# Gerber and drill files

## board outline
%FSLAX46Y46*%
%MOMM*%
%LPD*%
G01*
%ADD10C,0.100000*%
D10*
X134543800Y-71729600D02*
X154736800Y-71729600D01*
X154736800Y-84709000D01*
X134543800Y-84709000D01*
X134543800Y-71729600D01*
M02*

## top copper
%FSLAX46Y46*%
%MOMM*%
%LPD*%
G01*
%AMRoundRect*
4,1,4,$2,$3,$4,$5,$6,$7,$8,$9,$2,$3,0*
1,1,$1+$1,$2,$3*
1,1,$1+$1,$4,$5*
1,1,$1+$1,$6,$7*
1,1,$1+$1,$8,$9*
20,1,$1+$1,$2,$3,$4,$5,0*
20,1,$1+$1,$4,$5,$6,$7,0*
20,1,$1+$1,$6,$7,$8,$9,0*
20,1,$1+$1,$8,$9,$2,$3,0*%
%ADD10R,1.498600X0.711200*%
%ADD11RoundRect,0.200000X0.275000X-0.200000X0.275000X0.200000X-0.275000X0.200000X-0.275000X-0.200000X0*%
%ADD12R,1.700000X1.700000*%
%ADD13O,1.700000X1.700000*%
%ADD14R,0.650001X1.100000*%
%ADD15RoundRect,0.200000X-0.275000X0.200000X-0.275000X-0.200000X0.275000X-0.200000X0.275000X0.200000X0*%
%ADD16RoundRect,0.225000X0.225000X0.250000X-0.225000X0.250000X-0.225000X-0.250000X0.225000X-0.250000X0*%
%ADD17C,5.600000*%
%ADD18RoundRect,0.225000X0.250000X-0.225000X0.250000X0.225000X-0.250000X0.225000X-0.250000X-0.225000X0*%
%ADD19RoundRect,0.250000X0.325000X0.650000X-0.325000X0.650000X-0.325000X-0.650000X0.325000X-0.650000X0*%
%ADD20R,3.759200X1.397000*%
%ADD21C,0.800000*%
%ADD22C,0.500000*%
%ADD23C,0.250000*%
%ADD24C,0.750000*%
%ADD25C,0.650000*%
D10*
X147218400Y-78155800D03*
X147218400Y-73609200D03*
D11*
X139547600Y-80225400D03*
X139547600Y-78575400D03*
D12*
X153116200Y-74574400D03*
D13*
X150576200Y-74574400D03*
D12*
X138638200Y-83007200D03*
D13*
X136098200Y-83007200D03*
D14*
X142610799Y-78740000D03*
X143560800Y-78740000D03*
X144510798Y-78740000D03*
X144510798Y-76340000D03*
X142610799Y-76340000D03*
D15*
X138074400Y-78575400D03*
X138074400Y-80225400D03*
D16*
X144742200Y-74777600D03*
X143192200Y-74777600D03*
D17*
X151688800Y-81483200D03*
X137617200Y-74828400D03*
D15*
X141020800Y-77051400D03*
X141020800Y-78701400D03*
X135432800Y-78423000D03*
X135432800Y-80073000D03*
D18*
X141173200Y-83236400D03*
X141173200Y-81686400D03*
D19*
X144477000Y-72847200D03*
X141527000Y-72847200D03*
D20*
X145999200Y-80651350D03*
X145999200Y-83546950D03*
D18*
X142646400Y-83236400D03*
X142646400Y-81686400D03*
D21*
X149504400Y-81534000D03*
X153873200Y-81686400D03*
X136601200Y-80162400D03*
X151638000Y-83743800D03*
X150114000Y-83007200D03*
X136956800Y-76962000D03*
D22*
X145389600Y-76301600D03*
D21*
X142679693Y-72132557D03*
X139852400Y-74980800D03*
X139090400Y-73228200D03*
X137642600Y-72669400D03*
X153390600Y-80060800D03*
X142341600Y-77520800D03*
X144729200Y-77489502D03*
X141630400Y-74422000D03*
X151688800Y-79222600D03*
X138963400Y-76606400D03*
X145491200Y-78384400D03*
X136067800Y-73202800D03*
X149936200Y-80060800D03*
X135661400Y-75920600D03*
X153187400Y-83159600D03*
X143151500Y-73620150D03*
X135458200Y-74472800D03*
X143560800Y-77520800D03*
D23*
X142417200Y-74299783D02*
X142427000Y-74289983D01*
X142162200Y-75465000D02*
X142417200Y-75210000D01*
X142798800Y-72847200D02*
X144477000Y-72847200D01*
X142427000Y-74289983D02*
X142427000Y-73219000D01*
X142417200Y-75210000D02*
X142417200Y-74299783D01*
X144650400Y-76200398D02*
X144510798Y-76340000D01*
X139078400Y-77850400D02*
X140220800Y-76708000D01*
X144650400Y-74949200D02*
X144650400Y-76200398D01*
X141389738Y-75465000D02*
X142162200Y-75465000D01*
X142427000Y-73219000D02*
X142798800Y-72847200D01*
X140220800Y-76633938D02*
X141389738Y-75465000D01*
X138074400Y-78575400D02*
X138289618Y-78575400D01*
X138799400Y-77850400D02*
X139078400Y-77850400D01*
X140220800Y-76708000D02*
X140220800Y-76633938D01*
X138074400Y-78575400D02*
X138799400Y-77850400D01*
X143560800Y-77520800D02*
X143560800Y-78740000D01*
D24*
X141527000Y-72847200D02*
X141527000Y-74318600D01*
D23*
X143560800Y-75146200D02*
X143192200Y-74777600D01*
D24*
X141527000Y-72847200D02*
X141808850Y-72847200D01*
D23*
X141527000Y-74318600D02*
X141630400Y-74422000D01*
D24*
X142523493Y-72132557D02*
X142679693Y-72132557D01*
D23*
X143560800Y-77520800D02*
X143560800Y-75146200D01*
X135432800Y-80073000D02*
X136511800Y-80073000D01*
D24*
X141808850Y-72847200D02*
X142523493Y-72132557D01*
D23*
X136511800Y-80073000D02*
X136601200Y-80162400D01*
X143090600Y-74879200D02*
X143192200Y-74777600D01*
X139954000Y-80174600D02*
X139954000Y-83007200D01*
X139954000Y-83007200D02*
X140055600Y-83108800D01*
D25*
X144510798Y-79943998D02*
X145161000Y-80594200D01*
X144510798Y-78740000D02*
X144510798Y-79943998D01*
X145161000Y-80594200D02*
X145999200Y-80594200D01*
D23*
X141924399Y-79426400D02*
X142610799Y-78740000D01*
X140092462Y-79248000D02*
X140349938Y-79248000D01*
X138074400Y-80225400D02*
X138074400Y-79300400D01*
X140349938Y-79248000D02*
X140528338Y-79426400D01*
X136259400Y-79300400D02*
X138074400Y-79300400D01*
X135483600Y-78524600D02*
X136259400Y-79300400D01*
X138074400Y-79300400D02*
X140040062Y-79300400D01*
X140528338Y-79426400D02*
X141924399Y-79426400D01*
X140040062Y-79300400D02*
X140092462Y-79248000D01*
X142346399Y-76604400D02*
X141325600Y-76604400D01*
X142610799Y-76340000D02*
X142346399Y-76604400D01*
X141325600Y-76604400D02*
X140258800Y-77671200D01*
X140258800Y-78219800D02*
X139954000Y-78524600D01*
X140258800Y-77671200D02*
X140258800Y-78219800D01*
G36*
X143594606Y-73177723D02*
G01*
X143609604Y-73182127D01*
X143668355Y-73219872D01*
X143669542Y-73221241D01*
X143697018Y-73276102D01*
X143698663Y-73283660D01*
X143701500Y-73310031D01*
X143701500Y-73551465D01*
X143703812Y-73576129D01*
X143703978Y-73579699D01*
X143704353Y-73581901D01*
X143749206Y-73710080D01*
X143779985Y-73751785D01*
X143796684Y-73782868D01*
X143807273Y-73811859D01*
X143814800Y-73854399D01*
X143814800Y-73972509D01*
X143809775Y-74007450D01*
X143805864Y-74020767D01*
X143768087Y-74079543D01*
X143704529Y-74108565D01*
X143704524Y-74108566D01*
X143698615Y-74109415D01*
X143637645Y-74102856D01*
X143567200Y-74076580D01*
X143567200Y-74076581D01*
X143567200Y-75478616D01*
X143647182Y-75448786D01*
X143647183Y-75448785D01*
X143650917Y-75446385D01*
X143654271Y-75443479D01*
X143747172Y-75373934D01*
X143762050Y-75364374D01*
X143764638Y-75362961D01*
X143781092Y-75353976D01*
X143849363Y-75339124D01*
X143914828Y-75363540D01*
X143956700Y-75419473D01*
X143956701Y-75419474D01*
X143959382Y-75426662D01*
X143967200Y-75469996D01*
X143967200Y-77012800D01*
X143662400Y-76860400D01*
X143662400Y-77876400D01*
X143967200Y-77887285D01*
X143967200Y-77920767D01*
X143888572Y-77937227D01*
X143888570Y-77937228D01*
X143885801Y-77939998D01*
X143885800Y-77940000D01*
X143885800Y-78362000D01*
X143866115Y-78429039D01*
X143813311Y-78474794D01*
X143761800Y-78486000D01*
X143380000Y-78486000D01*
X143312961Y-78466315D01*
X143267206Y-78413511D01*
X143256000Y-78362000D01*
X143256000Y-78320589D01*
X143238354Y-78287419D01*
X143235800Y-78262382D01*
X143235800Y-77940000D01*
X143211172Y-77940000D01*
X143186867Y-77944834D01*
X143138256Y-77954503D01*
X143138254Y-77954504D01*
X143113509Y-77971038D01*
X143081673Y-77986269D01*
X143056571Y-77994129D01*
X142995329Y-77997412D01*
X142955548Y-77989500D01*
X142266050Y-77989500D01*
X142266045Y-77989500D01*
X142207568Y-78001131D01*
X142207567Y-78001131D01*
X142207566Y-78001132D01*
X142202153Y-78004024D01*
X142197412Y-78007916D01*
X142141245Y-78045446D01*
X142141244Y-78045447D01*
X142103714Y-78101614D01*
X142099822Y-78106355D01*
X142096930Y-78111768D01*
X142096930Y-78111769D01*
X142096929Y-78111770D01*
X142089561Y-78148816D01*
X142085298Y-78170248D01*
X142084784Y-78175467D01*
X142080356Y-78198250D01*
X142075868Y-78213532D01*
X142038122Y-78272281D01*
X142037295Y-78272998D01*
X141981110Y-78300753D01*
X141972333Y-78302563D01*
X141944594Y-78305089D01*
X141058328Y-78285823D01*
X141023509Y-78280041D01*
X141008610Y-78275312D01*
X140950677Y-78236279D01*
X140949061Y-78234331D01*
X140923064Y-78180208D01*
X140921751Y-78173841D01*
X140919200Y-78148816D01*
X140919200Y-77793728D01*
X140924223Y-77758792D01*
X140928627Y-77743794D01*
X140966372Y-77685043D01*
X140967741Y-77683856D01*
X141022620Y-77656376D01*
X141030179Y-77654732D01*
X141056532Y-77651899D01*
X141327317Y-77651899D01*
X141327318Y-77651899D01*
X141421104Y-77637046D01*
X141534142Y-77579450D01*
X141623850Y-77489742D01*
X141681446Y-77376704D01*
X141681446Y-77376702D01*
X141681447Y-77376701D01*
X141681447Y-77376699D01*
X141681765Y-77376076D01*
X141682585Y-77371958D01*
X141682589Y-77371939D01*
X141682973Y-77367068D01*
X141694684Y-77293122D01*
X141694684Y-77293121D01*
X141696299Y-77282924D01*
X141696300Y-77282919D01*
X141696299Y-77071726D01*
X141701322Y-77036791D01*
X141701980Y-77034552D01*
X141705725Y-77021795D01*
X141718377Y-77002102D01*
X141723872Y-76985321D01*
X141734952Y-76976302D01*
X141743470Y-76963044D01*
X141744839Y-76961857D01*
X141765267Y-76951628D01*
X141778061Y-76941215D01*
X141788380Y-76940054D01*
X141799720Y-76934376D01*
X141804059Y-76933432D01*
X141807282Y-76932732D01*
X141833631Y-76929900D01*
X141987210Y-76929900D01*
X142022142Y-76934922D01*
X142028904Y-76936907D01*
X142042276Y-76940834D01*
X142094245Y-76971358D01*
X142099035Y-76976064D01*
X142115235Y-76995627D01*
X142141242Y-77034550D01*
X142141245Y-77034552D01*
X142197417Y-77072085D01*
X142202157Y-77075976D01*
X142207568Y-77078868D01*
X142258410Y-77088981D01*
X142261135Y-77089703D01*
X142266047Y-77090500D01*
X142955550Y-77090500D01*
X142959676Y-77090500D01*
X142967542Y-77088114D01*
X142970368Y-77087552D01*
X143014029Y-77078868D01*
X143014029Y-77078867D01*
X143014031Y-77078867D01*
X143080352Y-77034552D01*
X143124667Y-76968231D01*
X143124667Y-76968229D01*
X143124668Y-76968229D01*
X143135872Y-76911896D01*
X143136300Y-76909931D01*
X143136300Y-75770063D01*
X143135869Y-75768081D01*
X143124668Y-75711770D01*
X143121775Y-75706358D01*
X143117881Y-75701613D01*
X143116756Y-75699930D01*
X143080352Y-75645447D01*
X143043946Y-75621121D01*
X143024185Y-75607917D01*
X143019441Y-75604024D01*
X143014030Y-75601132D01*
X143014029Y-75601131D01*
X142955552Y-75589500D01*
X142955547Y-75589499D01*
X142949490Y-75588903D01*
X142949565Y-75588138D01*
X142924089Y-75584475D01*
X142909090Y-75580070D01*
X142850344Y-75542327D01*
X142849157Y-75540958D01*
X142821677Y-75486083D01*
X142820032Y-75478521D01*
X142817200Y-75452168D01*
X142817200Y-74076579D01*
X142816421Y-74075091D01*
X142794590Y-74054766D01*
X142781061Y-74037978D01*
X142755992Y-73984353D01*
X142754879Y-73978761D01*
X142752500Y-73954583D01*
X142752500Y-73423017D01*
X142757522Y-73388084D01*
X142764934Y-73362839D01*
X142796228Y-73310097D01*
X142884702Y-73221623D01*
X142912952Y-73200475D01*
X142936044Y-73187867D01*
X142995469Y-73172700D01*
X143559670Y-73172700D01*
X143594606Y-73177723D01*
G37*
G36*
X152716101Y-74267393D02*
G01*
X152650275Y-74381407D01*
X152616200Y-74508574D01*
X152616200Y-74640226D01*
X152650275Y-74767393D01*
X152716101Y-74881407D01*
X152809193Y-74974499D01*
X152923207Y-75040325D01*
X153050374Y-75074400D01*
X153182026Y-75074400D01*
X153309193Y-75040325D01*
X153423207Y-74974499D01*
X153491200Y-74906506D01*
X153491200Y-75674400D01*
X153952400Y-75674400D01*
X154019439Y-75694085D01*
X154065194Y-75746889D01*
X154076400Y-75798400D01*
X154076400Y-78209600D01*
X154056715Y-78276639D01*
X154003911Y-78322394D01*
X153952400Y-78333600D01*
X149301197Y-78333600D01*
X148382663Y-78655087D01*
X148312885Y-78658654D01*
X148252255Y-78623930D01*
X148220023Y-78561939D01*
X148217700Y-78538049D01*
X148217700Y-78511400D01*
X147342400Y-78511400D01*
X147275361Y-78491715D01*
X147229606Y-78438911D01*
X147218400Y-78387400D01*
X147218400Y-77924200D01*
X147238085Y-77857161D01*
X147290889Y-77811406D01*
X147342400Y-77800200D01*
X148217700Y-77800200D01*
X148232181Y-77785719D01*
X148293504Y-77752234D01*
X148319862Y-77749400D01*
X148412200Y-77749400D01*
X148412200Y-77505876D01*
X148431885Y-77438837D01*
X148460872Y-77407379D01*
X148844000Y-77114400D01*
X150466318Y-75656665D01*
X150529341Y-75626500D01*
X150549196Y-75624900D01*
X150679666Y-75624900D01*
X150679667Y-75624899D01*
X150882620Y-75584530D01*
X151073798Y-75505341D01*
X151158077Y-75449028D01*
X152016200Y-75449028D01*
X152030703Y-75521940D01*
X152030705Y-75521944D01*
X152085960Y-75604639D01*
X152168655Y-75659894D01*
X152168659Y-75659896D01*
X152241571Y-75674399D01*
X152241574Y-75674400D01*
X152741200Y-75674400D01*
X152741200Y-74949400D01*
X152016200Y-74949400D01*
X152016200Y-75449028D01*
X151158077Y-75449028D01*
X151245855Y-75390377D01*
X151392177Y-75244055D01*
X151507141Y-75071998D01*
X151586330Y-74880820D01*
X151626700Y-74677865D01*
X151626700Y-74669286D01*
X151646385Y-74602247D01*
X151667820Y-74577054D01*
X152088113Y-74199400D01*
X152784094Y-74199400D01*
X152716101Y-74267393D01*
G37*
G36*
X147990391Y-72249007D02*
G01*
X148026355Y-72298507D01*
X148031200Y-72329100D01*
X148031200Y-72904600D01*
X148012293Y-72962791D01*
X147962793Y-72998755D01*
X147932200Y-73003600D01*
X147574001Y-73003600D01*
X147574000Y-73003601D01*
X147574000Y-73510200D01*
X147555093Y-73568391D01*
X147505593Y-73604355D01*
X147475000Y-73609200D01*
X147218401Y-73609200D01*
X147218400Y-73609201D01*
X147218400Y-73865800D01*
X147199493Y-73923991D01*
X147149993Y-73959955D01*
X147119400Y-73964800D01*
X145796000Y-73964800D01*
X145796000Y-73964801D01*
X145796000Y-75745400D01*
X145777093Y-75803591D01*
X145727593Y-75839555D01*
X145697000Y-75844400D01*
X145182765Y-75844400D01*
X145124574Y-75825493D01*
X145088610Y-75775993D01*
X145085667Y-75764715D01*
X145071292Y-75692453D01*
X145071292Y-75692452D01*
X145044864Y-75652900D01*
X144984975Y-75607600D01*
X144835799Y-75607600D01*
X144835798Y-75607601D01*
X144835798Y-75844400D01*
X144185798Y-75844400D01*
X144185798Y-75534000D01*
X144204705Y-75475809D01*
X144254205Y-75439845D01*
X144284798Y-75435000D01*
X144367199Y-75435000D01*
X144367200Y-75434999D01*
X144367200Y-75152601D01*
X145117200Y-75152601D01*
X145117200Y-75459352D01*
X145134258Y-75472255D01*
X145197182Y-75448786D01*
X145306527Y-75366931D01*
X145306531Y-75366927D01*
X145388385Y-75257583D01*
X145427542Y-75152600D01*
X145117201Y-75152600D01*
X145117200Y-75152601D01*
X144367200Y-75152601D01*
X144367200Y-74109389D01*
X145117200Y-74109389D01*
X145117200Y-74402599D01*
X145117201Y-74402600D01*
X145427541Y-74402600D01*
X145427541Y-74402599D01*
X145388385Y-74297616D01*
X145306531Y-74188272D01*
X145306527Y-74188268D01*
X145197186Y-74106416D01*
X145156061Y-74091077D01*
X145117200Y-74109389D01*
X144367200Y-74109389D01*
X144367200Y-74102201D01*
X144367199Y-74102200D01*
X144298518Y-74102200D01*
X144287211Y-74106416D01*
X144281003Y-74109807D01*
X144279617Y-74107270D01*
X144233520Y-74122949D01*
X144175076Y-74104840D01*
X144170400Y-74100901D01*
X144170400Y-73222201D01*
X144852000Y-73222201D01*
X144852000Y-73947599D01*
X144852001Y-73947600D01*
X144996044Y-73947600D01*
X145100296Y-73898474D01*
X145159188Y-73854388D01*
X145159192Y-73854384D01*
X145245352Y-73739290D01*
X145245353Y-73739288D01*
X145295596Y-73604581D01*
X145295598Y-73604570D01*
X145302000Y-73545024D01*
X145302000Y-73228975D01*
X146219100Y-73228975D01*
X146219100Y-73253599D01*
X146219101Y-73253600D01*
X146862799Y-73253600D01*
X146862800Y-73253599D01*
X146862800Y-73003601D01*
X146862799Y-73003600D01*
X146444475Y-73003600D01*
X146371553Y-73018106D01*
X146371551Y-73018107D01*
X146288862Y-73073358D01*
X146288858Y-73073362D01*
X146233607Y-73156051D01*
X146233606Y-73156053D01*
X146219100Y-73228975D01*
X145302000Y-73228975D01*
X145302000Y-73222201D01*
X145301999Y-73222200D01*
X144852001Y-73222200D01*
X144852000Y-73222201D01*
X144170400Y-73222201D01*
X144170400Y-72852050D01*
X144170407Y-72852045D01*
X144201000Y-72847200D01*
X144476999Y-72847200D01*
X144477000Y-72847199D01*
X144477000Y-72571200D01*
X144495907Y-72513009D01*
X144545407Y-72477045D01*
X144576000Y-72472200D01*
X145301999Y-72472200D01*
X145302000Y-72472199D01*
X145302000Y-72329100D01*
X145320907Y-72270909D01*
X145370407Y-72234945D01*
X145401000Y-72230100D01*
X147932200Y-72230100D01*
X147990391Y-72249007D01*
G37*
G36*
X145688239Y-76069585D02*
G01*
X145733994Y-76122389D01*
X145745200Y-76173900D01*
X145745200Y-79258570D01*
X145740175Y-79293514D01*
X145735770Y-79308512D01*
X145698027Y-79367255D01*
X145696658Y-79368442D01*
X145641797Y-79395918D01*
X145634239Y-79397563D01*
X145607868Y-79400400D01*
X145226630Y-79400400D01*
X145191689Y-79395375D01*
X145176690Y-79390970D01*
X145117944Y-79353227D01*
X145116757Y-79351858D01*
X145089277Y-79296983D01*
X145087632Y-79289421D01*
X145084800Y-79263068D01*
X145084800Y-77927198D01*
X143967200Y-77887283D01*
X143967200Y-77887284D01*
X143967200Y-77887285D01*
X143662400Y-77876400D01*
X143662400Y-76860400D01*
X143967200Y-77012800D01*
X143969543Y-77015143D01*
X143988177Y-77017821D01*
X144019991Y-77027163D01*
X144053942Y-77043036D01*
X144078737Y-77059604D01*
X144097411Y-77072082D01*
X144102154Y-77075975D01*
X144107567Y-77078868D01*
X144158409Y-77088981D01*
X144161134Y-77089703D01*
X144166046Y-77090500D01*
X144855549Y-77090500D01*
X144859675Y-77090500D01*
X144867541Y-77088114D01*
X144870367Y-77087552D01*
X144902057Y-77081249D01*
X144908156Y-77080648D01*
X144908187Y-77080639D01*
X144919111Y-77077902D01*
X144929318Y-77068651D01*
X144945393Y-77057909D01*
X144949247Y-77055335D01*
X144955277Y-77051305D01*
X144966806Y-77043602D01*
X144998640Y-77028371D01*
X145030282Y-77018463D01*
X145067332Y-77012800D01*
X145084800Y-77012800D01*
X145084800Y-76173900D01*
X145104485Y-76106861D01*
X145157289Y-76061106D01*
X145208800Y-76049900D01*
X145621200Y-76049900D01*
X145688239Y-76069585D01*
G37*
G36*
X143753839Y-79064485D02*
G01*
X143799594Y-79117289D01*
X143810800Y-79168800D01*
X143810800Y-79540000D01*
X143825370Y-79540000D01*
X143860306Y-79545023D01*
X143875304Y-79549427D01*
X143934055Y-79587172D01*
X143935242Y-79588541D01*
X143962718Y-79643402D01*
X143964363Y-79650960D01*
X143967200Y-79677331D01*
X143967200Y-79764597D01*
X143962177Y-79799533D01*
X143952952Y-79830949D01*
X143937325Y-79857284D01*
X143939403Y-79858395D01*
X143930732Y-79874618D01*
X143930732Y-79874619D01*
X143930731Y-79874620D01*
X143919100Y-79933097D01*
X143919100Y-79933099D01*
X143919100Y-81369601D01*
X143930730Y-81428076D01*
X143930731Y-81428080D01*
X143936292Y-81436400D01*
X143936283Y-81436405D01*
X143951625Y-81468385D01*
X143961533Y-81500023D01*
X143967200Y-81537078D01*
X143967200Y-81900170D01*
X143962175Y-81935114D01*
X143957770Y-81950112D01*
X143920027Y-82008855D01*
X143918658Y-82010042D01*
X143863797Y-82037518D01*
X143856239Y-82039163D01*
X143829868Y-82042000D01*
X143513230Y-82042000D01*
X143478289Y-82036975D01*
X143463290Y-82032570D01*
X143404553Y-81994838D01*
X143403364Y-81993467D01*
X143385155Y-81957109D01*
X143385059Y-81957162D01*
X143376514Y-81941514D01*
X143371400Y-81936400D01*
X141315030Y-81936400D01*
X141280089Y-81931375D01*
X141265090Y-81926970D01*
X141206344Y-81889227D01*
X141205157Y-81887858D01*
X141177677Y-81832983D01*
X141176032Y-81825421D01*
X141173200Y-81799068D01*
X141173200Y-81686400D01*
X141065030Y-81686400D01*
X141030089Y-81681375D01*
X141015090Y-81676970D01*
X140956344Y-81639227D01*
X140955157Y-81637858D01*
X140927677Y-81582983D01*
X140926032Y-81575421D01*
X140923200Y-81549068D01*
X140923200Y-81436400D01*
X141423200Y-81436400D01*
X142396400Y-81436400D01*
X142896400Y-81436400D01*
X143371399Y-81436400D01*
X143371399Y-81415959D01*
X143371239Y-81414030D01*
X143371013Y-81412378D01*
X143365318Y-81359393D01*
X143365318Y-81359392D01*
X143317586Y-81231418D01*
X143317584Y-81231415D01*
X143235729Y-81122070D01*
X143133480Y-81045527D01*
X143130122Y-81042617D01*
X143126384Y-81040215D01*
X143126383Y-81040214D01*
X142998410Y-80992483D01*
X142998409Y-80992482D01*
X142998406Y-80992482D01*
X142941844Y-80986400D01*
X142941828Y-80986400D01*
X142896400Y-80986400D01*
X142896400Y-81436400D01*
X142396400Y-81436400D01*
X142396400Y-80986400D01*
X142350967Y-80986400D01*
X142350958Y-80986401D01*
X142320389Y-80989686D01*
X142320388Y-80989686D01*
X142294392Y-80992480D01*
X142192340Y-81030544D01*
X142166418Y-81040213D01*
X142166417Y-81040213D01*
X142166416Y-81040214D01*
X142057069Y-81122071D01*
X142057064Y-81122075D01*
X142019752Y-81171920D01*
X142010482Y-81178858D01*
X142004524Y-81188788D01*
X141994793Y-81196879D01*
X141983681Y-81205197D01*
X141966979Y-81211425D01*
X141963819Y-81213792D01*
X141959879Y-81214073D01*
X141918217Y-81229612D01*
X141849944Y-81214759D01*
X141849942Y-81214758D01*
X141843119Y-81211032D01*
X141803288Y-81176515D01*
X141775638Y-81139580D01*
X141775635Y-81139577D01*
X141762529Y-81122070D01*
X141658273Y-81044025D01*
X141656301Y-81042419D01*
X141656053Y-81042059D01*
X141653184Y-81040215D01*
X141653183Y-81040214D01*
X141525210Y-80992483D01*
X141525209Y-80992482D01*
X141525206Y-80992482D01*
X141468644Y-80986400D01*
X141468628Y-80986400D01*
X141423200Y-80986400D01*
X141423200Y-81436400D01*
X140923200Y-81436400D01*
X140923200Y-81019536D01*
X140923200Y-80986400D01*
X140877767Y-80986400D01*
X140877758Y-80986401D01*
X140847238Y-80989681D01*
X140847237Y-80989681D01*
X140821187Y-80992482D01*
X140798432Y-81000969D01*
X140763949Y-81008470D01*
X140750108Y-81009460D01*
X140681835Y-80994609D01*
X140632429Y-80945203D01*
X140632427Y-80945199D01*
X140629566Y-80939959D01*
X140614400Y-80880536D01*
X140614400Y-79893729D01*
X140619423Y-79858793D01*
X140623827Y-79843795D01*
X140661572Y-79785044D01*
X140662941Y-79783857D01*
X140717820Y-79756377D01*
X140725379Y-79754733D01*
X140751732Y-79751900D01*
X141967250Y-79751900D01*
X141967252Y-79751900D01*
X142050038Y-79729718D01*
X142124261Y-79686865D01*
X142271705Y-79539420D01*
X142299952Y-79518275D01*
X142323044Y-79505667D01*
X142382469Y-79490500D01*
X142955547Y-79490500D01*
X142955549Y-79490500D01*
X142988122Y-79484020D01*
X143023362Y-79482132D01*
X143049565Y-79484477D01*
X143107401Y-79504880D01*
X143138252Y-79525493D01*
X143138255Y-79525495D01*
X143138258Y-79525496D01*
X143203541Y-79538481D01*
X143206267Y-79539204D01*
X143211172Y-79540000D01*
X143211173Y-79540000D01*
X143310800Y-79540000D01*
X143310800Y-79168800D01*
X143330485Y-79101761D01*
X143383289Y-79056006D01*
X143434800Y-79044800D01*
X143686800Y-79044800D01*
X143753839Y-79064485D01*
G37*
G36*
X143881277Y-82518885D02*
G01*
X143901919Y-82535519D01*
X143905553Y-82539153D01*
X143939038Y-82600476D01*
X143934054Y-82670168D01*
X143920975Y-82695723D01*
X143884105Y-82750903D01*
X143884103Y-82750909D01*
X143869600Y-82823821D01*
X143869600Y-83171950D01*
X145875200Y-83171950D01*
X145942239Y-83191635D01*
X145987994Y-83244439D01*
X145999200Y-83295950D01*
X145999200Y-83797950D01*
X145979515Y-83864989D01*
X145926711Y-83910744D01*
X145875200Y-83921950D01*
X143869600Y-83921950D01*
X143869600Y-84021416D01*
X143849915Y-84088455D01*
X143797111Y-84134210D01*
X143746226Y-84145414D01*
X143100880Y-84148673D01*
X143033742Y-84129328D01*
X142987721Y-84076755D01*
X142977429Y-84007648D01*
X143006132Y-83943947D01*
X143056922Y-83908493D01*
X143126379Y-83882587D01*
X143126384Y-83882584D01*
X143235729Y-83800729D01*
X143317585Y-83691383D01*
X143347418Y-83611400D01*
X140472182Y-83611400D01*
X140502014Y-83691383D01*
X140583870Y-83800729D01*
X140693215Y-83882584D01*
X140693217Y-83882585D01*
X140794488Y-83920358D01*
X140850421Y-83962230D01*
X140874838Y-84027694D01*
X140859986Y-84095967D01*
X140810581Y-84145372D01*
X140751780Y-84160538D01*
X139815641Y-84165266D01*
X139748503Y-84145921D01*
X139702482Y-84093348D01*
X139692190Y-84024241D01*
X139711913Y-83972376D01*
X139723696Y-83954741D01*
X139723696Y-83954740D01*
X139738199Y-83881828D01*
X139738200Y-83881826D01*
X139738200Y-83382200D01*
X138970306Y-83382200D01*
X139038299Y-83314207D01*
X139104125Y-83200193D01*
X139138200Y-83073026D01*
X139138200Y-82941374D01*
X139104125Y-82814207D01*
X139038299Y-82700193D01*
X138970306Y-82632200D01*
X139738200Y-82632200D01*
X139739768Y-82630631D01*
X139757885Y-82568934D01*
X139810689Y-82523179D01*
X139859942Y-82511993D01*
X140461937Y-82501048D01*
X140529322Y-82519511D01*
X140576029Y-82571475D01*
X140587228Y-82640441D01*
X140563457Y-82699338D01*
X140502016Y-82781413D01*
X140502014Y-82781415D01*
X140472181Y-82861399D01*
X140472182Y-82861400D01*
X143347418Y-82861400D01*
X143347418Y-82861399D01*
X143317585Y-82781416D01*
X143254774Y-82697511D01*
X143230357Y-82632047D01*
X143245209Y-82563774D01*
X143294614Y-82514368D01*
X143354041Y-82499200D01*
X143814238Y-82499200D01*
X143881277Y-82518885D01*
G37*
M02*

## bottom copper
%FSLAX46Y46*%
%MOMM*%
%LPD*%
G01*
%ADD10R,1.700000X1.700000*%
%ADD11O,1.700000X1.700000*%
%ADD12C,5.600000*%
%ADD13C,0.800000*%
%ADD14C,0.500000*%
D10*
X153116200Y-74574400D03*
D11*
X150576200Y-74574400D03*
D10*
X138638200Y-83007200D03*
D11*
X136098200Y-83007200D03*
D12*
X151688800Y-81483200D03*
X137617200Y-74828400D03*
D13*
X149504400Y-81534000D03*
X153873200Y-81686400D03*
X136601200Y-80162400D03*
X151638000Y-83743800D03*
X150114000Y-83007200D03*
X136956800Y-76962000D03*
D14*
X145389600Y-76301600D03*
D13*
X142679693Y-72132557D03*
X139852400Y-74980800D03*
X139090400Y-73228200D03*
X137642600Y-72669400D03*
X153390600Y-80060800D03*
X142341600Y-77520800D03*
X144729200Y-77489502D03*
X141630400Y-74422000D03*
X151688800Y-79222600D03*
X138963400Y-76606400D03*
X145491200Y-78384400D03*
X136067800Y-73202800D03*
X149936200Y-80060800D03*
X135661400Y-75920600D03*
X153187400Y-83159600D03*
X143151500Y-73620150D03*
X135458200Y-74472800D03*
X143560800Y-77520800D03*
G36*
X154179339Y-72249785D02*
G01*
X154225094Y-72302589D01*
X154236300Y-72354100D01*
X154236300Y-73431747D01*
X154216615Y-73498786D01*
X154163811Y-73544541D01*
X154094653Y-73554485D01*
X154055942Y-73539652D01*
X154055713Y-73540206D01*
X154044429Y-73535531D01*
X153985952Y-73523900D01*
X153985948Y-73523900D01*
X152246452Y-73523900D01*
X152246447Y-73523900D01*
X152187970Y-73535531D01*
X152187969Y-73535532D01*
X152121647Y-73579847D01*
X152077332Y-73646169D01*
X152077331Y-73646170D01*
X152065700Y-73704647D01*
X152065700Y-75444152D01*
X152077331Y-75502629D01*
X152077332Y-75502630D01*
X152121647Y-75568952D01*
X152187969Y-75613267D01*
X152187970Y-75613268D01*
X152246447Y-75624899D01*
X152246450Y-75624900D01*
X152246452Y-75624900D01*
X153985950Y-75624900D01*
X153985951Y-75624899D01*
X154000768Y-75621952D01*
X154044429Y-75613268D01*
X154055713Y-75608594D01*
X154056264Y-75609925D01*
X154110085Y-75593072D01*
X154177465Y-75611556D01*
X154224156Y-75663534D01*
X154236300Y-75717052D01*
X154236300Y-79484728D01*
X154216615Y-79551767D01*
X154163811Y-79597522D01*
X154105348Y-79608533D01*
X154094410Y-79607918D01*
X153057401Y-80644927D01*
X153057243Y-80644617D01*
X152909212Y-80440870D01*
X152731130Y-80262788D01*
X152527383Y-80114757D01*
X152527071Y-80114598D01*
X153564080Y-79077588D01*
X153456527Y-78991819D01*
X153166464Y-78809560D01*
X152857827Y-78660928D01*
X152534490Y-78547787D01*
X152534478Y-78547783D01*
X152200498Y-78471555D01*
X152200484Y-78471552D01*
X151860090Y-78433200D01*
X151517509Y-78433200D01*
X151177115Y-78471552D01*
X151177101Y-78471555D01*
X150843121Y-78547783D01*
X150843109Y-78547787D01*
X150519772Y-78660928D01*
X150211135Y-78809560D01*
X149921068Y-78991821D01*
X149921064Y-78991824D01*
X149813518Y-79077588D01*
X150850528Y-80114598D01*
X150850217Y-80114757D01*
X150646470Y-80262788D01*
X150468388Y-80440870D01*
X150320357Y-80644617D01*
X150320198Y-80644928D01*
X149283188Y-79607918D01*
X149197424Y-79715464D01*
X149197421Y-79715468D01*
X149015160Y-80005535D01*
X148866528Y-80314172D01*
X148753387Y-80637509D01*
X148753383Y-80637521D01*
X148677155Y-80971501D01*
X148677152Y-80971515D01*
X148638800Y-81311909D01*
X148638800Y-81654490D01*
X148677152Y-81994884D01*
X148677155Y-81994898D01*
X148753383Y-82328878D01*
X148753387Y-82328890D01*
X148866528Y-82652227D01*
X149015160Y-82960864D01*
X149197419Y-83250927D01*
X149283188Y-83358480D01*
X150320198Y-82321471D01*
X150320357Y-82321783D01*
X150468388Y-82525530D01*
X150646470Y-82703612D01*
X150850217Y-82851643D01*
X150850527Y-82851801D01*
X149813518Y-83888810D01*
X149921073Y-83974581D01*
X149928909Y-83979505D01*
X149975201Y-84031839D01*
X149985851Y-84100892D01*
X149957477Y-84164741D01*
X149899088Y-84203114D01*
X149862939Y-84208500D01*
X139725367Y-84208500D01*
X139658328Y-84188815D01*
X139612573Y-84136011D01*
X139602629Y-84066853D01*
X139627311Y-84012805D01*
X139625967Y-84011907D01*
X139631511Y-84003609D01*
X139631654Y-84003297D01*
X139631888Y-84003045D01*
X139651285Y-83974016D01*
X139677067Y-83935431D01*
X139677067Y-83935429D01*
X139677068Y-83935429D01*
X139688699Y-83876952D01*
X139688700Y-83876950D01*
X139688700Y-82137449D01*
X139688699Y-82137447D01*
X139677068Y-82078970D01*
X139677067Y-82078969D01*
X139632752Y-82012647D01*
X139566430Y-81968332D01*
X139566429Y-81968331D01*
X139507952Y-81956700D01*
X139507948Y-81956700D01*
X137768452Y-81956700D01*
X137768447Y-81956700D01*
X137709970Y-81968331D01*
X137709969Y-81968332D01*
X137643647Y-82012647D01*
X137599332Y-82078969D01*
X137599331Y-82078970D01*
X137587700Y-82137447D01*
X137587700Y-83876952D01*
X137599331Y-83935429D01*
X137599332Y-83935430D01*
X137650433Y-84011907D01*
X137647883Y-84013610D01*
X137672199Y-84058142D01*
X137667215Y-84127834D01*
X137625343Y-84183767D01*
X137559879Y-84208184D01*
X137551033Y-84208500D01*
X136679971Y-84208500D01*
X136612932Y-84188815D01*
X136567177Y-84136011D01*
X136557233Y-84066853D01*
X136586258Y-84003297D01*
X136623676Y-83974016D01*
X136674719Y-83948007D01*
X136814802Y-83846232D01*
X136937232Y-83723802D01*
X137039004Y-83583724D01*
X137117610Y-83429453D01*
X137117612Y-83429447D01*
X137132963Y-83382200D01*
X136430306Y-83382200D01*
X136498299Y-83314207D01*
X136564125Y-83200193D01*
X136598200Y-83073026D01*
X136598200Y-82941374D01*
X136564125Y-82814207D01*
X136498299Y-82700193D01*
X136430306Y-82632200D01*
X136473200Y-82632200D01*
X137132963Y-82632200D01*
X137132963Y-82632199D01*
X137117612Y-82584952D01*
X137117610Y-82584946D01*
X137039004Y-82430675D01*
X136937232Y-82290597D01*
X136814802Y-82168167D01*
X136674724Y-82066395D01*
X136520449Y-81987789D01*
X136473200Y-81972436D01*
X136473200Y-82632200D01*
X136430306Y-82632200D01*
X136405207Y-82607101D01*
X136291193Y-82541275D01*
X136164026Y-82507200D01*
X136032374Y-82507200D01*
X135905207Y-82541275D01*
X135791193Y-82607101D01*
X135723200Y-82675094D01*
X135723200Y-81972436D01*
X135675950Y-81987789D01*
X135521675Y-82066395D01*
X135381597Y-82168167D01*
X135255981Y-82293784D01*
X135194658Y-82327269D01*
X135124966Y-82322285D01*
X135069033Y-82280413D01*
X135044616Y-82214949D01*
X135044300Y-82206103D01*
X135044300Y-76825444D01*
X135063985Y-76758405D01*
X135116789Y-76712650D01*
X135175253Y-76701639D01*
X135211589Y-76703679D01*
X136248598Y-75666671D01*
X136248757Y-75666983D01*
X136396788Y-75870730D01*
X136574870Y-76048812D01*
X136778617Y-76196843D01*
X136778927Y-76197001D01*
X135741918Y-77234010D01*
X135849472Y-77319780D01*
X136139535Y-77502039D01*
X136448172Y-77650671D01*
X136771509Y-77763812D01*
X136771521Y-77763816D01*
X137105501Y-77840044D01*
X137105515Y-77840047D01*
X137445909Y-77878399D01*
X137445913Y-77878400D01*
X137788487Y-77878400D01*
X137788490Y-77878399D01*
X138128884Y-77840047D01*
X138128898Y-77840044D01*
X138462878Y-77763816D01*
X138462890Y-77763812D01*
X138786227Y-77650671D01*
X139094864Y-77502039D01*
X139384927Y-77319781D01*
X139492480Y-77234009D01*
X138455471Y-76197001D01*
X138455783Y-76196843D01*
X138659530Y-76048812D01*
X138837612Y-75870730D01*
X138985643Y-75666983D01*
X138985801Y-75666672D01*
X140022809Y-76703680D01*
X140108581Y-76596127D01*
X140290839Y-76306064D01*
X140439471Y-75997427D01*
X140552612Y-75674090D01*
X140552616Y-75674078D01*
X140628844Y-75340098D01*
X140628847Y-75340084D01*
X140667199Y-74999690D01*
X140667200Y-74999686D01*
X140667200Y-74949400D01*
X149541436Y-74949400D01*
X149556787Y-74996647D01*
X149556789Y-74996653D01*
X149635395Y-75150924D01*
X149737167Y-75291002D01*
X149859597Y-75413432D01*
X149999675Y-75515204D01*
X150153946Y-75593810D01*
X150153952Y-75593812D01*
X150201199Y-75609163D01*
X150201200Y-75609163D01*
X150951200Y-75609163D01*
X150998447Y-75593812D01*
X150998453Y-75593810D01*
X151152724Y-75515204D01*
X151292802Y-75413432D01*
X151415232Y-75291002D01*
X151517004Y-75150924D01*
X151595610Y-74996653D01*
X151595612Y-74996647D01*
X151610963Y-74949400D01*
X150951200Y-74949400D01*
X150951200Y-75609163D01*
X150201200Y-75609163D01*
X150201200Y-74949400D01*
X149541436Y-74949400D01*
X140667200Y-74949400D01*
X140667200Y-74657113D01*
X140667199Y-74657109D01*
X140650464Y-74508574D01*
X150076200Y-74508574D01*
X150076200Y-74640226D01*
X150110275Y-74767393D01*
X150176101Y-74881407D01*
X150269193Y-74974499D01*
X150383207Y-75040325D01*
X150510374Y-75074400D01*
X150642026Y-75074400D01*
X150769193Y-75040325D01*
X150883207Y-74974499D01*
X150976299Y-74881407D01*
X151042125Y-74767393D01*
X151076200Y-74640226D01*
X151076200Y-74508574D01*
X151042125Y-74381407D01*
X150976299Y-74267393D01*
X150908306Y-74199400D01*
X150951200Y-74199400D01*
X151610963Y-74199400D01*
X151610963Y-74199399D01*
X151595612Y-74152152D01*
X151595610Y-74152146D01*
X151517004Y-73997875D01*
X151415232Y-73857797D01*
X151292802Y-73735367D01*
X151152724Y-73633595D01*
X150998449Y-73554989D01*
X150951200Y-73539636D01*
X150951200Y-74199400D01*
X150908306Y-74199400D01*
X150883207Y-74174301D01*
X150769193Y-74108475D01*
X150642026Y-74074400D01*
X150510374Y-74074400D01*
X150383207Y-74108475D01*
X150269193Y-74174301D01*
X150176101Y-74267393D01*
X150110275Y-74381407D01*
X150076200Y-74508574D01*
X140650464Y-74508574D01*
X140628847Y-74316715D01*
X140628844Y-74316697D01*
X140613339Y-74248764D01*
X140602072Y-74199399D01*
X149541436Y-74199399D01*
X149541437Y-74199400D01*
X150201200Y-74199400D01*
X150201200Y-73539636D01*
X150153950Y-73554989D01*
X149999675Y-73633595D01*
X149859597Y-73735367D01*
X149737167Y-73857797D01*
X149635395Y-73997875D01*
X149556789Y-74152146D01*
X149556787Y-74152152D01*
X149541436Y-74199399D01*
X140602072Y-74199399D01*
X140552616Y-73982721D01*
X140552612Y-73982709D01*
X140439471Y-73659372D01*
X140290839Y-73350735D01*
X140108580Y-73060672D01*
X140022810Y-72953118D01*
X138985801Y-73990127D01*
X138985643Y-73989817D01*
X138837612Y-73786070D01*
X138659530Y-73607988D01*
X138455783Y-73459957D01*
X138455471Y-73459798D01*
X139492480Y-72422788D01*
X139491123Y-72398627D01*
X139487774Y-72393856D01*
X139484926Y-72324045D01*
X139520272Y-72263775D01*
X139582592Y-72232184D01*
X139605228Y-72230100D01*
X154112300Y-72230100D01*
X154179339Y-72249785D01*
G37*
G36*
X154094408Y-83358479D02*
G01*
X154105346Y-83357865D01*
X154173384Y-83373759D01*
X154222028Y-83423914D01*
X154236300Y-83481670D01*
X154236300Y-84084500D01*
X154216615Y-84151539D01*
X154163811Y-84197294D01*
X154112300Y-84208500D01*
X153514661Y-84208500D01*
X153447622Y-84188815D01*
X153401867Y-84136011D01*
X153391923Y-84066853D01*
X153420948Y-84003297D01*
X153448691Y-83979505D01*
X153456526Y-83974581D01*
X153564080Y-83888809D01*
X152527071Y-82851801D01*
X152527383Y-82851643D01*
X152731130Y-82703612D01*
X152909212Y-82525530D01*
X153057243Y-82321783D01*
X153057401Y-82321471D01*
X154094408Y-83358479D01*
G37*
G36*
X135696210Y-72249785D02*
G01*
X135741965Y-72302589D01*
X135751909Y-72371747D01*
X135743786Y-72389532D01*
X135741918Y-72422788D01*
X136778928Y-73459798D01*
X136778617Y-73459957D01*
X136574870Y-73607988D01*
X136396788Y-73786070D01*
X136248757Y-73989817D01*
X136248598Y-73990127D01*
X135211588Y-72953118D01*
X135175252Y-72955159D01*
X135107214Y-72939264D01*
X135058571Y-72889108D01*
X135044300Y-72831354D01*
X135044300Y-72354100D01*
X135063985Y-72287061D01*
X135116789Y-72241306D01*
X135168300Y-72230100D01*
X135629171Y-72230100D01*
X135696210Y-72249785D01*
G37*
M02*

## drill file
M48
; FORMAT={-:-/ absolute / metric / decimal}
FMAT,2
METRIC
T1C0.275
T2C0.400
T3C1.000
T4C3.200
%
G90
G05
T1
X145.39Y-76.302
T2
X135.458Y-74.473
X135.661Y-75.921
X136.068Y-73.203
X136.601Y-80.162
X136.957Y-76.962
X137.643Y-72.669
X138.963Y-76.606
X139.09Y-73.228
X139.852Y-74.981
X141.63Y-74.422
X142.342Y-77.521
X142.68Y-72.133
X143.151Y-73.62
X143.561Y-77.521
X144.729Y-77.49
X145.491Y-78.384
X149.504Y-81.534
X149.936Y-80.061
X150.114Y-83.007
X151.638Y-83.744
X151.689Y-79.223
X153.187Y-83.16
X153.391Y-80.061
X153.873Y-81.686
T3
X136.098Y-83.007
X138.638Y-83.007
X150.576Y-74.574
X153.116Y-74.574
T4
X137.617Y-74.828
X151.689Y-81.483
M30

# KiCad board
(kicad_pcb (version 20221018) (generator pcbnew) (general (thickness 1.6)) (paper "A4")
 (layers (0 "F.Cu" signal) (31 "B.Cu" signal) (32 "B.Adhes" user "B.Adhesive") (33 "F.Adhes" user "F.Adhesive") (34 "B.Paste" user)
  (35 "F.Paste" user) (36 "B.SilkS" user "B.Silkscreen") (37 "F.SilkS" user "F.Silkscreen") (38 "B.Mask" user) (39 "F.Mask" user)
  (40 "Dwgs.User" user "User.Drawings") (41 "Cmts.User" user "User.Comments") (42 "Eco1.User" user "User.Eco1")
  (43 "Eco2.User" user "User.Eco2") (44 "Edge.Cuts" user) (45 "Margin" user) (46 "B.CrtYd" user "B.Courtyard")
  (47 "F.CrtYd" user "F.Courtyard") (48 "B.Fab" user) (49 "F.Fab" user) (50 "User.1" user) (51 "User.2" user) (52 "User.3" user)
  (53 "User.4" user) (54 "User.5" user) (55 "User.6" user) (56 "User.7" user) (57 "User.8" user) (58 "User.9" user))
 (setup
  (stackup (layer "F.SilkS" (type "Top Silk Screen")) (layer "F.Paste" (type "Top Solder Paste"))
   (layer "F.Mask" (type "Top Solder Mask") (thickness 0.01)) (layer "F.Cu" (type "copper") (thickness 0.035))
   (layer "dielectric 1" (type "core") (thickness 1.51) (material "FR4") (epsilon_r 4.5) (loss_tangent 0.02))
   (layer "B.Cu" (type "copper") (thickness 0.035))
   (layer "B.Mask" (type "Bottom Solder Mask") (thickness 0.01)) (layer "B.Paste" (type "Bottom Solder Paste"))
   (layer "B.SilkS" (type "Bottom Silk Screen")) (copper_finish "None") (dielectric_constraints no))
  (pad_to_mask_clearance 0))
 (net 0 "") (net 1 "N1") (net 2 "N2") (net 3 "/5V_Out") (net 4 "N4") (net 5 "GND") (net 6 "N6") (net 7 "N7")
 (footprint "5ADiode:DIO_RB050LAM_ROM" (layer "F.Cu") (at 147.2184 75.8825 90)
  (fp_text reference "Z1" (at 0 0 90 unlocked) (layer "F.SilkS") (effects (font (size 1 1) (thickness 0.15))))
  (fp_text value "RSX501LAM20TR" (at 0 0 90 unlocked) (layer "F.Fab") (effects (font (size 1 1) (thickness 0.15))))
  (pad "1" smd rect (at -2.2733 0 90) (size 0.7112 1.4986) (layers "F.Cu" "F.Paste" "F.Mask") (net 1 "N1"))
  (pad "2" smd rect (at 2.2733 0 90) (size 0.7112 1.4986) (layers "F.Cu" "F.Paste" "F.Mask") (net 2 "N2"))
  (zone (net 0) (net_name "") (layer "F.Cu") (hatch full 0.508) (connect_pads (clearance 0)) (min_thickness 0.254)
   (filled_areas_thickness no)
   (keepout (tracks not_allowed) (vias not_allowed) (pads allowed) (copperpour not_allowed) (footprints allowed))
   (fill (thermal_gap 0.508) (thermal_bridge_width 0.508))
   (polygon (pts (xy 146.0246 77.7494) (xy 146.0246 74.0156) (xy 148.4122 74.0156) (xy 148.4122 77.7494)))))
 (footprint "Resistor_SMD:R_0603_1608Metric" (layer "F.Cu") (at 139.5476 79.4004 90)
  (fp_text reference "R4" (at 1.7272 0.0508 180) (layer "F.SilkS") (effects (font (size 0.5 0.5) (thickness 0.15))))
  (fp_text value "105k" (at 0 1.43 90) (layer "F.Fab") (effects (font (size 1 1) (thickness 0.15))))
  (pad "1" smd roundrect (at -0.825 0 90) (size 0.8 0.95) (layers "F.Cu" "F.Paste" "F.Mask") (roundrect_rratio 0.25) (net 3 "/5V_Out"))
  (pad "2" smd roundrect (at 0.825 0 90) (size 0.8 0.95) (layers "F.Cu" "F.Paste" "F.Mask") (roundrect_rratio 0.25) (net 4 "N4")))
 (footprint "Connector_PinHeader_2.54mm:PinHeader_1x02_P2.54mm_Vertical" (layer "F.Cu") (at 153.1162 74.5744 -90)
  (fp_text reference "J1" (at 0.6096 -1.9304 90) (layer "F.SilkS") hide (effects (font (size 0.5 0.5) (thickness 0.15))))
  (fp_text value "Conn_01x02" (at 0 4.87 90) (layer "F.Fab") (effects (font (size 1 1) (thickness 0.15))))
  (pad "1" thru_hole rect (at 0 0 270) (size 1.7 1.7) (drill 1) (layers "*.Cu" "*.Mask") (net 1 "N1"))
  (pad "2" thru_hole oval (at 0 2.54 270) (size 1.7 1.7) (drill 1) (layers "*.Cu" "*.Mask") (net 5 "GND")))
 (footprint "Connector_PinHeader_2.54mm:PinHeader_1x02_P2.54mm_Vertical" (layer "F.Cu") (at 138.6382 83.0072 -90)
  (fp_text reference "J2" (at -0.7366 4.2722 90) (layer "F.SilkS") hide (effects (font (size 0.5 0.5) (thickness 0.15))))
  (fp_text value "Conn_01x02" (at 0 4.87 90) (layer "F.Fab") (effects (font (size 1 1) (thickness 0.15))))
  (pad "1" thru_hole rect (at 0 0 270) (size 1.7 1.7) (drill 1) (layers "*.Cu" "*.Mask") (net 3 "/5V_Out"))
  (pad "2" thru_hole oval (at 0 2.54 270) (size 1.7 1.7) (drill 1) (layers "*.Cu" "*.Mask") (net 5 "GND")))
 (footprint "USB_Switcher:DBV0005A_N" (layer "F.Cu") (at 143.5608 77.54 90)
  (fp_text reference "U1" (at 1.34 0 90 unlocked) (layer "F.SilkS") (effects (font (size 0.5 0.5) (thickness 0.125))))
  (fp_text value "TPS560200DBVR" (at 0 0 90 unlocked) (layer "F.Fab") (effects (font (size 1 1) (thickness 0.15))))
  (pad "1" smd rect (at -1.2 -0.950001 180) (size 0.650001 1.1) (layers "F.Cu" "F.Paste" "F.Mask") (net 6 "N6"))
  (pad "2" smd rect (at -1.2 0 180) (size 0.650001 1.1) (layers "F.Cu" "F.Paste" "F.Mask") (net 5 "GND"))
  (pad "3" smd rect (at -1.2 0.949998 180) (size 0.650001 1.1) (layers "F.Cu" "F.Paste" "F.Mask") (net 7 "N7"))
  (pad "4" smd rect (at 1.2 0.949998 180) (size 0.650001 1.1) (layers "F.Cu" "F.Paste" "F.Mask") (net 2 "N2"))
  (pad "5" smd rect (at 1.2 -0.950001 180) (size 0.650001 1.1) (layers "F.Cu" "F.Paste" "F.Mask") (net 4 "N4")))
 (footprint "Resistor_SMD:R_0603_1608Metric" (layer "F.Cu") (at 138.0744 79.4004 -90)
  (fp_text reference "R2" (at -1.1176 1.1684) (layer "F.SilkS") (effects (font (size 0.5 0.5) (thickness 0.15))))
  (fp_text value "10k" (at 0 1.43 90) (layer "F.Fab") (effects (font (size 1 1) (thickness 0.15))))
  (pad "1" smd roundrect (at -0.825 0 270) (size 0.8 0.95) (layers "F.Cu" "F.Paste" "F.Mask") (roundrect_rratio 0.25) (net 2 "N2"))
  (pad "2" smd roundrect (at 0.825 0 270) (size 0.8 0.95) (layers "F.Cu" "F.Paste" "F.Mask") (roundrect_rratio 0.25) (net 6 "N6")))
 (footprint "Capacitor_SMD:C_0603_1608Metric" (layer "F.Cu") (at 143.9672 74.7776 180)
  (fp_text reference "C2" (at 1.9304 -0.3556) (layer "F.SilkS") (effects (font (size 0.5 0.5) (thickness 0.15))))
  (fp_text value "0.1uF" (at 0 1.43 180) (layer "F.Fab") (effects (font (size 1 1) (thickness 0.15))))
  (pad "1" smd roundrect (at -0.775 0 180) (size 0.9 0.95) (layers "F.Cu" "F.Paste" "F.Mask") (roundrect_rratio 0.25) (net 2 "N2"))
  (pad "2" smd roundrect (at 0.775 0 180) (size 0.9 0.95) (layers "F.Cu" "F.Paste" "F.Mask") (roundrect_rratio 0.25) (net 5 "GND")))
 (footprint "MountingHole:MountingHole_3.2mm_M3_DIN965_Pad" (layer "F.Cu") (at 151.6888 81.4832)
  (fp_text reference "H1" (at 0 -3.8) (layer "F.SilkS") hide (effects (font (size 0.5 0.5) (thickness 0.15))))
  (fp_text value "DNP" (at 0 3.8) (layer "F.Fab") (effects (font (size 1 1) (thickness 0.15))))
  (pad "1" thru_hole circle (at 0 0) (size 5.6 5.6) (drill 3.2) (layers "*.Cu" "*.Mask") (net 5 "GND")))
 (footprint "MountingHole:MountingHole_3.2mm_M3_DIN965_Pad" (layer "F.Cu") (at 137.6172 74.8284)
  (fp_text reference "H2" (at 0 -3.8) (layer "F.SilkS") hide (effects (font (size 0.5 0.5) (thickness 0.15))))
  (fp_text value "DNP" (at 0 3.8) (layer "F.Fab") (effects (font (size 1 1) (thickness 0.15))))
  (pad "1" thru_hole circle (at 0 0) (size 5.6 5.6) (drill 3.2) (layers "*.Cu" "*.Mask") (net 5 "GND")))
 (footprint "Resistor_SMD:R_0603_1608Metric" (layer "F.Cu") (at 141.0208 77.8764 -90)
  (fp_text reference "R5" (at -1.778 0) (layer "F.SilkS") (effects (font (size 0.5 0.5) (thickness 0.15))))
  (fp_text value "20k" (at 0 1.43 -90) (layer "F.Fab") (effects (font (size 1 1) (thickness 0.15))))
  (pad "1" smd roundrect (at -0.825 0 270) (size 0.8 0.95) (layers "F.Cu" "F.Paste" "F.Mask") (roundrect_rratio 0.25) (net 4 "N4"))
  (pad "2" smd roundrect (at 0.825 0 270) (size 0.8 0.95) (layers "F.Cu" "F.Paste" "F.Mask") (roundrect_rratio 0.25) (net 5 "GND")))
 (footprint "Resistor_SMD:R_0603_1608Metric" (layer "F.Cu") (at 135.4328 79.248 -90)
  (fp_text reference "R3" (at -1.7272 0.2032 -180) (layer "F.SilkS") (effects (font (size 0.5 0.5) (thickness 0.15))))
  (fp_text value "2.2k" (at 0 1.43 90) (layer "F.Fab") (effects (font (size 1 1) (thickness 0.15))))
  (pad "1" smd roundrect (at -0.825 0 270) (size 0.8 0.95) (layers "F.Cu" "F.Paste" "F.Mask") (roundrect_rratio 0.25) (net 6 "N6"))
  (pad "2" smd roundrect (at 0.825 0 270) (size 0.8 0.95) (layers "F.Cu" "F.Paste" "F.Mask") (roundrect_rratio 0.25) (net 5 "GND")))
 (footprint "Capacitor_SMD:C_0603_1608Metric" (layer "F.Cu") (at 141.1732 82.4614 90)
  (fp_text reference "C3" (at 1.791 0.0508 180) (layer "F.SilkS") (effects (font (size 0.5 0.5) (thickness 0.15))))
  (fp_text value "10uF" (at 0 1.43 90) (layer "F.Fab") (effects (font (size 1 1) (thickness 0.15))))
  (pad "1" smd roundrect (at -0.775 0 90) (size 0.9 0.95) (layers "F.Cu" "F.Paste" "F.Mask") (roundrect_rratio 0.25) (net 3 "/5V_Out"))
  (pad "2" smd roundrect (at 0.775 0 90) (size 0.9 0.95) (layers "F.Cu" "F.Paste" "F.Mask") (roundrect_rratio 0.25) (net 5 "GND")))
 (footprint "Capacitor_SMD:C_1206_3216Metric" (layer "F.Cu") (at 143.002 72.8472 180)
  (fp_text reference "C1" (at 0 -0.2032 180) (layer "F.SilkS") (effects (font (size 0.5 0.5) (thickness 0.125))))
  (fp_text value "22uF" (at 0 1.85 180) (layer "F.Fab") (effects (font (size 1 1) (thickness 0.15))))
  (pad "1" smd roundrect (at -1.475 0 180) (size 1.15 1.8) (layers "F.Cu" "F.Paste" "F.Mask") (roundrect_rratio 0.2173913043) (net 2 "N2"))
  (pad "2" smd roundrect (at 1.475 0 180) (size 1.15 1.8) (layers "F.Cu" "F.Paste" "F.Mask") (roundrect_rratio 0.2173913043) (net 5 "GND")))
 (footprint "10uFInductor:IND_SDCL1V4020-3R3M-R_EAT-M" (layer "F.Cu") (at 145.9992 82.09915 -90)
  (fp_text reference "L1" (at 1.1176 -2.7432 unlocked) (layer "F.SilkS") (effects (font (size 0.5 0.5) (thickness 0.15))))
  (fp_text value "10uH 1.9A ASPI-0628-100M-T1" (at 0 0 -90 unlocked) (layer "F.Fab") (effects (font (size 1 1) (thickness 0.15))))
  (pad "1" smd rect (at -1.4478 0 270) (size 1.397 3.7592) (layers "F.Cu" "F.Paste" "F.Mask") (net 7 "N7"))
  (pad "2" smd rect (at 1.4478 0 270) (size 1.397 3.7592) (layers "F.Cu" "F.Paste" "F.Mask") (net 3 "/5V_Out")))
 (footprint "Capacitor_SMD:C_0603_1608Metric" (layer "F.Cu") (at 142.6464 82.4614 90)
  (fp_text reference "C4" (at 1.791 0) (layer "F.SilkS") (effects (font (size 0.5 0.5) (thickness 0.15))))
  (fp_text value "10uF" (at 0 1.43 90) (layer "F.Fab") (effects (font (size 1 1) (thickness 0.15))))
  (pad "1" smd roundrect (at -0.775 0 90) (size 0.9 0.95) (layers "F.Cu" "F.Paste" "F.Mask") (roundrect_rratio 0.25) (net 3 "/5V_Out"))
  (pad "2" smd roundrect (at 0.775 0 90) (size 0.9 0.95) (layers "F.Cu" "F.Paste" "F.Mask") (roundrect_rratio 0.25) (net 5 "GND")))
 (gr_rect (start 134.5438 71.7296) (end 154.7368 84.709) (stroke (width 0.1) (type default)) (fill none) (layer "Edge.Cuts"))
 (segment (start 142.4172 74.299783) (end 142.427 74.289983) (width 0.25) (layer "F.Cu") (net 2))
 (segment (start 142.1622 75.465) (end 142.4172 75.21) (width 0.25) (layer "F.Cu") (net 2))
 (segment (start 142.7988 72.8472) (end 144.477 72.8472) (width 0.25) (layer "F.Cu") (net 2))
 (segment (start 142.427 74.289983) (end 142.427 73.219) (width 0.25) (layer "F.Cu") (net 2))
 (segment (start 142.4172 75.21) (end 142.4172 74.299783) (width 0.25) (layer "F.Cu") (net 2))
 (segment (start 144.6504 76.200398) (end 144.510798 76.34) (width 0.25) (layer "F.Cu") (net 2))
 (segment (start 139.0784 77.8504) (end 140.2208 76.708) (width 0.25) (layer "F.Cu") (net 2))
 (segment (start 144.6504 74.9492) (end 144.6504 76.200398) (width 0.25) (layer "F.Cu") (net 2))
 (segment (start 141.389738 75.465) (end 142.1622 75.465) (width 0.25) (layer "F.Cu") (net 2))
 (segment (start 142.427 73.219) (end 142.7988 72.8472) (width 0.25) (layer "F.Cu") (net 2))
 (segment (start 140.2208 76.633938) (end 141.389738 75.465) (width 0.25) (layer "F.Cu") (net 2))
 (segment (start 138.0744 78.5754) (end 138.289618 78.5754) (width 0.25) (layer "F.Cu") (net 2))
 (segment (start 138.7994 77.8504) (end 139.0784 77.8504) (width 0.25) (layer "F.Cu") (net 2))
 (segment (start 140.2208 76.708) (end 140.2208 76.633938) (width 0.25) (layer "F.Cu") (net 2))
 (segment (start 138.0744 78.5754) (end 138.7994 77.8504) (width 0.25) (layer "F.Cu") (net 2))
 (segment (start 143.5608 77.5208) (end 143.5608 78.74) (width 0.25) (layer "F.Cu") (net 5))
 (segment (start 141.527 72.8472) (end 141.527 74.3186) (width 0.75) (layer "F.Cu") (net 5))
 (segment (start 143.5608 75.1462) (end 143.1922 74.7776) (width 0.25) (layer "F.Cu") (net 5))
 (segment (start 141.527 72.8472) (end 141.80885 72.8472) (width 0.75) (layer "F.Cu") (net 5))
 (segment (start 141.527 74.3186) (end 141.6304 74.422) (width 0.25) (layer "F.Cu") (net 5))
 (segment (start 142.523493 72.132557) (end 142.679693 72.132557) (width 0.75) (layer "F.Cu") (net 5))
 (segment (start 143.5608 77.5208) (end 143.5608 75.1462) (width 0.25) (layer "F.Cu") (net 5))
 (segment (start 135.4328 80.073) (end 136.5118 80.073) (width 0.25) (layer "F.Cu") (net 5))
 (segment (start 141.80885 72.8472) (end 142.523493 72.132557) (width 0.75) (layer "F.Cu") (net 5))
 (segment (start 136.5118 80.073) (end 136.6012 80.1624) (width 0.25) (layer "F.Cu") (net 5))
 (segment (start 143.0906 74.8792) (end 143.1922 74.7776) (width 0.25) (layer "F.Cu") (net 5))
 (via (at 149.5044 81.534) (size 0.8) (drill 0.4) (layers "F.Cu" "B.Cu") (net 5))
 (via (at 153.8732 81.6864) (size 0.8) (drill 0.4) (layers "F.Cu" "B.Cu") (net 5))
 (via (at 136.6012 80.1624) (size 0.8) (drill 0.4) (layers "F.Cu" "B.Cu") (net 5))
 (via (at 151.638 83.7438) (size 0.8) (drill 0.4) (layers "F.Cu" "B.Cu") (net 5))
 (via (at 150.114 83.0072) (size 0.8) (drill 0.4) (layers "F.Cu" "B.Cu") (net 5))
 (via (at 136.9568 76.962) (size 0.8) (drill 0.4) (layers "F.Cu" "B.Cu") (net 5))
 (via (at 145.3896 76.3016) (size 0.5) (drill 0.275) (layers "F.Cu" "B.Cu") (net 5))
 (via (at 142.679693 72.132557) (size 0.8) (drill 0.4) (layers "F.Cu" "B.Cu") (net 5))
 (via (at 139.8524 74.9808) (size 0.8) (drill 0.4) (layers "F.Cu" "B.Cu") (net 5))
 (via (at 139.0904 73.2282) (size 0.8) (drill 0.4) (layers "F.Cu" "B.Cu") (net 5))
 (via (at 137.6426 72.6694) (size 0.8) (drill 0.4) (layers "F.Cu" "B.Cu") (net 5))
 (via (at 153.3906 80.0608) (size 0.8) (drill 0.4) (layers "F.Cu" "B.Cu") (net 5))
 (via (at 142.3416 77.5208) (size 0.8) (drill 0.4) (layers "F.Cu" "B.Cu") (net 5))
 (via (at 144.7292 77.489502) (size 0.8) (drill 0.4) (layers "F.Cu" "B.Cu") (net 5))
 (via (at 141.6304 74.422) (size 0.8) (drill 0.4) (layers "F.Cu" "B.Cu") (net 5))
 (via (at 151.6888 79.2226) (size 0.8) (drill 0.4) (layers "F.Cu" "B.Cu") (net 5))
 (via (at 138.9634 76.6064) (size 0.8) (drill 0.4) (layers "F.Cu" "B.Cu") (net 5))
 (via (at 145.4912 78.3844) (size 0.8) (drill 0.4) (layers "F.Cu" "B.Cu") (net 5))
 (via (at 136.0678 73.2028) (size 0.8) (drill 0.4) (layers "F.Cu" "B.Cu") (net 5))
 (via (at 149.9362 80.0608) (size 0.8) (drill 0.4) (layers "F.Cu" "B.Cu") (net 5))
 (via (at 135.6614 75.9206) (size 0.8) (drill 0.4) (layers "F.Cu" "B.Cu") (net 5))
 (via (at 153.1874 83.1596) (size 0.8) (drill 0.4) (layers "F.Cu" "B.Cu") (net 5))
 (via (at 143.1515 73.62015) (size 0.8) (drill 0.4) (layers "F.Cu" "B.Cu") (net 5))
 (via (at 135.4582 74.4728) (size 0.8) (drill 0.4) (layers "F.Cu" "B.Cu") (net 5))
 (via (at 143.5608 77.5208) (size 0.8) (drill 0.4) (layers "F.Cu" "B.Cu") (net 5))
 (segment (start 139.954 80.1746) (end 139.954 83.0072) (width 0.25) (layer "F.Cu") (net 3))
 (segment (start 139.954 83.0072) (end 140.0556 83.1088) (width 0.25) (layer "F.Cu") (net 3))
 (segment (start 144.510798 79.943998) (end 145.161 80.5942) (width 0.65) (layer "F.Cu") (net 7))
 (segment (start 144.510798 78.74) (end 144.510798 79.943998) (width 0.65) (layer "F.Cu") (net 7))
 (segment (start 145.161 80.5942) (end 145.9992 80.5942) (width 0.65) (layer "F.Cu") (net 7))
 (segment (start 141.924399 79.4264) (end 142.610799 78.74) (width 0.25) (layer "F.Cu") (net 6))
 (segment (start 140.092462 79.248) (end 140.349938 79.248) (width 0.25) (layer "F.Cu") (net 6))
 (segment (start 138.0744 80.2254) (end 138.0744 79.3004) (width 0.25) (layer "F.Cu") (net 6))
 (segment (start 140.349938 79.248) (end 140.528338 79.4264) (width 0.25) (layer "F.Cu") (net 6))
 (segment (start 136.2594 79.3004) (end 138.0744 79.3004) (width 0.25) (layer "F.Cu") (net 6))
 (segment (start 135.4836 78.5246) (end 136.2594 79.3004) (width 0.25) (layer "F.Cu") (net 6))
 (segment (start 138.0744 79.3004) (end 140.040062 79.3004) (width 0.25) (layer "F.Cu") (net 6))
 (segment (start 140.528338 79.4264) (end 141.924399 79.4264) (width 0.25) (layer "F.Cu") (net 6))
 (segment (start 140.040062 79.3004) (end 140.092462 79.248) (width 0.25) (layer "F.Cu") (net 6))
 (segment (start 142.346399 76.6044) (end 141.3256 76.6044) (width 0.25) (layer "F.Cu") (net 4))
 (segment (start 142.610799 76.34) (end 142.346399 76.6044) (width 0.25) (layer "F.Cu") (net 4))
 (segment (start 141.3256 76.6044) (end 140.2588 77.6712) (width 0.25) (layer "F.Cu") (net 4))
 (segment (start 140.2588 78.2198) (end 139.954 78.5246) (width 0.25) (layer "F.Cu") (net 4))
 (segment (start 140.2588 77.6712) (end 140.2588 78.2198) (width 0.25) (layer "F.Cu") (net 4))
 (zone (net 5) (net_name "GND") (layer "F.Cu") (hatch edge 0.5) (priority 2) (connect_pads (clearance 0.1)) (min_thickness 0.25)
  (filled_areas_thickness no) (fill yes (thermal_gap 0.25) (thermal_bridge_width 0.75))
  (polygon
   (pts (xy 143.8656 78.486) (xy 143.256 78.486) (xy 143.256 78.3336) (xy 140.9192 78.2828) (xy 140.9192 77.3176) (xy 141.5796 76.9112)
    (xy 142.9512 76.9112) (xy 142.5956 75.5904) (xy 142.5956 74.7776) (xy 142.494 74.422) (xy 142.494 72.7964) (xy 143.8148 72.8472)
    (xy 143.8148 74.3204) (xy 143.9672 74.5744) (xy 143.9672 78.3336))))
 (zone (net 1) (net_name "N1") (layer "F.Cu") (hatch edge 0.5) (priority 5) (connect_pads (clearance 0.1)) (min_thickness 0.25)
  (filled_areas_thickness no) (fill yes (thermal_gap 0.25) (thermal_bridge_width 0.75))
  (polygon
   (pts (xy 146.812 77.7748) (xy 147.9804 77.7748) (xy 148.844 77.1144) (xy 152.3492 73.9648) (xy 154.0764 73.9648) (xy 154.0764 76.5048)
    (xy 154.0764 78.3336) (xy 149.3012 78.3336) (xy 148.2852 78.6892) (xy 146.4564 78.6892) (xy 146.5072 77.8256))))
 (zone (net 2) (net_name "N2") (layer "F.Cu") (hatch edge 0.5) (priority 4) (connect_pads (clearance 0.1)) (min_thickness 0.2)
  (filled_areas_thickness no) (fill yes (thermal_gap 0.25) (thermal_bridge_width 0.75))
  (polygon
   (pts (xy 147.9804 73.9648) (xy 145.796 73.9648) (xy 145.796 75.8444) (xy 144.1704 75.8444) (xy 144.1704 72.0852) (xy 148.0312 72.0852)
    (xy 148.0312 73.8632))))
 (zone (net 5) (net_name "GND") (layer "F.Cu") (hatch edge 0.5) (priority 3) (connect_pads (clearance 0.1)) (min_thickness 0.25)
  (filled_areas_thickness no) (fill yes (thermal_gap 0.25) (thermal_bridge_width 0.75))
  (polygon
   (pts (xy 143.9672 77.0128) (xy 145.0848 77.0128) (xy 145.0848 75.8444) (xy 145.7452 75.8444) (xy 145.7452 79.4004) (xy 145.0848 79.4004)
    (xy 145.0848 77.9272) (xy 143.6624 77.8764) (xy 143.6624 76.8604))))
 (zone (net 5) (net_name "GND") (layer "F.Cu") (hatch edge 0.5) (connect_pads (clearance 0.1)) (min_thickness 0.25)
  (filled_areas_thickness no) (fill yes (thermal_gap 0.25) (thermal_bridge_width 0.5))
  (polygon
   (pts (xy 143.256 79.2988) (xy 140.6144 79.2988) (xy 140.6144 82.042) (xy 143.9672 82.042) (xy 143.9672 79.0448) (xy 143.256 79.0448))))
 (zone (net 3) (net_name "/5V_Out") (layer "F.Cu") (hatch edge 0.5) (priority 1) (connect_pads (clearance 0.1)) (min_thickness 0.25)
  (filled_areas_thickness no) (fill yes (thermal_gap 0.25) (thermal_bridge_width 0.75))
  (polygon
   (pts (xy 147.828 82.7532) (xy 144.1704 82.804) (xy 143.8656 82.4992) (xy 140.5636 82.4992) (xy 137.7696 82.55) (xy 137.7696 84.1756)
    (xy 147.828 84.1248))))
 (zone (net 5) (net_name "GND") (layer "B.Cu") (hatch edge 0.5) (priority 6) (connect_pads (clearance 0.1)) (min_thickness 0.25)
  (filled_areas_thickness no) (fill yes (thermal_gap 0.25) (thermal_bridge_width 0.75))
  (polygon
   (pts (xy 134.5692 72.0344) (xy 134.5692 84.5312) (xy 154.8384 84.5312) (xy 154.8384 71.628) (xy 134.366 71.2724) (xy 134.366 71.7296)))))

